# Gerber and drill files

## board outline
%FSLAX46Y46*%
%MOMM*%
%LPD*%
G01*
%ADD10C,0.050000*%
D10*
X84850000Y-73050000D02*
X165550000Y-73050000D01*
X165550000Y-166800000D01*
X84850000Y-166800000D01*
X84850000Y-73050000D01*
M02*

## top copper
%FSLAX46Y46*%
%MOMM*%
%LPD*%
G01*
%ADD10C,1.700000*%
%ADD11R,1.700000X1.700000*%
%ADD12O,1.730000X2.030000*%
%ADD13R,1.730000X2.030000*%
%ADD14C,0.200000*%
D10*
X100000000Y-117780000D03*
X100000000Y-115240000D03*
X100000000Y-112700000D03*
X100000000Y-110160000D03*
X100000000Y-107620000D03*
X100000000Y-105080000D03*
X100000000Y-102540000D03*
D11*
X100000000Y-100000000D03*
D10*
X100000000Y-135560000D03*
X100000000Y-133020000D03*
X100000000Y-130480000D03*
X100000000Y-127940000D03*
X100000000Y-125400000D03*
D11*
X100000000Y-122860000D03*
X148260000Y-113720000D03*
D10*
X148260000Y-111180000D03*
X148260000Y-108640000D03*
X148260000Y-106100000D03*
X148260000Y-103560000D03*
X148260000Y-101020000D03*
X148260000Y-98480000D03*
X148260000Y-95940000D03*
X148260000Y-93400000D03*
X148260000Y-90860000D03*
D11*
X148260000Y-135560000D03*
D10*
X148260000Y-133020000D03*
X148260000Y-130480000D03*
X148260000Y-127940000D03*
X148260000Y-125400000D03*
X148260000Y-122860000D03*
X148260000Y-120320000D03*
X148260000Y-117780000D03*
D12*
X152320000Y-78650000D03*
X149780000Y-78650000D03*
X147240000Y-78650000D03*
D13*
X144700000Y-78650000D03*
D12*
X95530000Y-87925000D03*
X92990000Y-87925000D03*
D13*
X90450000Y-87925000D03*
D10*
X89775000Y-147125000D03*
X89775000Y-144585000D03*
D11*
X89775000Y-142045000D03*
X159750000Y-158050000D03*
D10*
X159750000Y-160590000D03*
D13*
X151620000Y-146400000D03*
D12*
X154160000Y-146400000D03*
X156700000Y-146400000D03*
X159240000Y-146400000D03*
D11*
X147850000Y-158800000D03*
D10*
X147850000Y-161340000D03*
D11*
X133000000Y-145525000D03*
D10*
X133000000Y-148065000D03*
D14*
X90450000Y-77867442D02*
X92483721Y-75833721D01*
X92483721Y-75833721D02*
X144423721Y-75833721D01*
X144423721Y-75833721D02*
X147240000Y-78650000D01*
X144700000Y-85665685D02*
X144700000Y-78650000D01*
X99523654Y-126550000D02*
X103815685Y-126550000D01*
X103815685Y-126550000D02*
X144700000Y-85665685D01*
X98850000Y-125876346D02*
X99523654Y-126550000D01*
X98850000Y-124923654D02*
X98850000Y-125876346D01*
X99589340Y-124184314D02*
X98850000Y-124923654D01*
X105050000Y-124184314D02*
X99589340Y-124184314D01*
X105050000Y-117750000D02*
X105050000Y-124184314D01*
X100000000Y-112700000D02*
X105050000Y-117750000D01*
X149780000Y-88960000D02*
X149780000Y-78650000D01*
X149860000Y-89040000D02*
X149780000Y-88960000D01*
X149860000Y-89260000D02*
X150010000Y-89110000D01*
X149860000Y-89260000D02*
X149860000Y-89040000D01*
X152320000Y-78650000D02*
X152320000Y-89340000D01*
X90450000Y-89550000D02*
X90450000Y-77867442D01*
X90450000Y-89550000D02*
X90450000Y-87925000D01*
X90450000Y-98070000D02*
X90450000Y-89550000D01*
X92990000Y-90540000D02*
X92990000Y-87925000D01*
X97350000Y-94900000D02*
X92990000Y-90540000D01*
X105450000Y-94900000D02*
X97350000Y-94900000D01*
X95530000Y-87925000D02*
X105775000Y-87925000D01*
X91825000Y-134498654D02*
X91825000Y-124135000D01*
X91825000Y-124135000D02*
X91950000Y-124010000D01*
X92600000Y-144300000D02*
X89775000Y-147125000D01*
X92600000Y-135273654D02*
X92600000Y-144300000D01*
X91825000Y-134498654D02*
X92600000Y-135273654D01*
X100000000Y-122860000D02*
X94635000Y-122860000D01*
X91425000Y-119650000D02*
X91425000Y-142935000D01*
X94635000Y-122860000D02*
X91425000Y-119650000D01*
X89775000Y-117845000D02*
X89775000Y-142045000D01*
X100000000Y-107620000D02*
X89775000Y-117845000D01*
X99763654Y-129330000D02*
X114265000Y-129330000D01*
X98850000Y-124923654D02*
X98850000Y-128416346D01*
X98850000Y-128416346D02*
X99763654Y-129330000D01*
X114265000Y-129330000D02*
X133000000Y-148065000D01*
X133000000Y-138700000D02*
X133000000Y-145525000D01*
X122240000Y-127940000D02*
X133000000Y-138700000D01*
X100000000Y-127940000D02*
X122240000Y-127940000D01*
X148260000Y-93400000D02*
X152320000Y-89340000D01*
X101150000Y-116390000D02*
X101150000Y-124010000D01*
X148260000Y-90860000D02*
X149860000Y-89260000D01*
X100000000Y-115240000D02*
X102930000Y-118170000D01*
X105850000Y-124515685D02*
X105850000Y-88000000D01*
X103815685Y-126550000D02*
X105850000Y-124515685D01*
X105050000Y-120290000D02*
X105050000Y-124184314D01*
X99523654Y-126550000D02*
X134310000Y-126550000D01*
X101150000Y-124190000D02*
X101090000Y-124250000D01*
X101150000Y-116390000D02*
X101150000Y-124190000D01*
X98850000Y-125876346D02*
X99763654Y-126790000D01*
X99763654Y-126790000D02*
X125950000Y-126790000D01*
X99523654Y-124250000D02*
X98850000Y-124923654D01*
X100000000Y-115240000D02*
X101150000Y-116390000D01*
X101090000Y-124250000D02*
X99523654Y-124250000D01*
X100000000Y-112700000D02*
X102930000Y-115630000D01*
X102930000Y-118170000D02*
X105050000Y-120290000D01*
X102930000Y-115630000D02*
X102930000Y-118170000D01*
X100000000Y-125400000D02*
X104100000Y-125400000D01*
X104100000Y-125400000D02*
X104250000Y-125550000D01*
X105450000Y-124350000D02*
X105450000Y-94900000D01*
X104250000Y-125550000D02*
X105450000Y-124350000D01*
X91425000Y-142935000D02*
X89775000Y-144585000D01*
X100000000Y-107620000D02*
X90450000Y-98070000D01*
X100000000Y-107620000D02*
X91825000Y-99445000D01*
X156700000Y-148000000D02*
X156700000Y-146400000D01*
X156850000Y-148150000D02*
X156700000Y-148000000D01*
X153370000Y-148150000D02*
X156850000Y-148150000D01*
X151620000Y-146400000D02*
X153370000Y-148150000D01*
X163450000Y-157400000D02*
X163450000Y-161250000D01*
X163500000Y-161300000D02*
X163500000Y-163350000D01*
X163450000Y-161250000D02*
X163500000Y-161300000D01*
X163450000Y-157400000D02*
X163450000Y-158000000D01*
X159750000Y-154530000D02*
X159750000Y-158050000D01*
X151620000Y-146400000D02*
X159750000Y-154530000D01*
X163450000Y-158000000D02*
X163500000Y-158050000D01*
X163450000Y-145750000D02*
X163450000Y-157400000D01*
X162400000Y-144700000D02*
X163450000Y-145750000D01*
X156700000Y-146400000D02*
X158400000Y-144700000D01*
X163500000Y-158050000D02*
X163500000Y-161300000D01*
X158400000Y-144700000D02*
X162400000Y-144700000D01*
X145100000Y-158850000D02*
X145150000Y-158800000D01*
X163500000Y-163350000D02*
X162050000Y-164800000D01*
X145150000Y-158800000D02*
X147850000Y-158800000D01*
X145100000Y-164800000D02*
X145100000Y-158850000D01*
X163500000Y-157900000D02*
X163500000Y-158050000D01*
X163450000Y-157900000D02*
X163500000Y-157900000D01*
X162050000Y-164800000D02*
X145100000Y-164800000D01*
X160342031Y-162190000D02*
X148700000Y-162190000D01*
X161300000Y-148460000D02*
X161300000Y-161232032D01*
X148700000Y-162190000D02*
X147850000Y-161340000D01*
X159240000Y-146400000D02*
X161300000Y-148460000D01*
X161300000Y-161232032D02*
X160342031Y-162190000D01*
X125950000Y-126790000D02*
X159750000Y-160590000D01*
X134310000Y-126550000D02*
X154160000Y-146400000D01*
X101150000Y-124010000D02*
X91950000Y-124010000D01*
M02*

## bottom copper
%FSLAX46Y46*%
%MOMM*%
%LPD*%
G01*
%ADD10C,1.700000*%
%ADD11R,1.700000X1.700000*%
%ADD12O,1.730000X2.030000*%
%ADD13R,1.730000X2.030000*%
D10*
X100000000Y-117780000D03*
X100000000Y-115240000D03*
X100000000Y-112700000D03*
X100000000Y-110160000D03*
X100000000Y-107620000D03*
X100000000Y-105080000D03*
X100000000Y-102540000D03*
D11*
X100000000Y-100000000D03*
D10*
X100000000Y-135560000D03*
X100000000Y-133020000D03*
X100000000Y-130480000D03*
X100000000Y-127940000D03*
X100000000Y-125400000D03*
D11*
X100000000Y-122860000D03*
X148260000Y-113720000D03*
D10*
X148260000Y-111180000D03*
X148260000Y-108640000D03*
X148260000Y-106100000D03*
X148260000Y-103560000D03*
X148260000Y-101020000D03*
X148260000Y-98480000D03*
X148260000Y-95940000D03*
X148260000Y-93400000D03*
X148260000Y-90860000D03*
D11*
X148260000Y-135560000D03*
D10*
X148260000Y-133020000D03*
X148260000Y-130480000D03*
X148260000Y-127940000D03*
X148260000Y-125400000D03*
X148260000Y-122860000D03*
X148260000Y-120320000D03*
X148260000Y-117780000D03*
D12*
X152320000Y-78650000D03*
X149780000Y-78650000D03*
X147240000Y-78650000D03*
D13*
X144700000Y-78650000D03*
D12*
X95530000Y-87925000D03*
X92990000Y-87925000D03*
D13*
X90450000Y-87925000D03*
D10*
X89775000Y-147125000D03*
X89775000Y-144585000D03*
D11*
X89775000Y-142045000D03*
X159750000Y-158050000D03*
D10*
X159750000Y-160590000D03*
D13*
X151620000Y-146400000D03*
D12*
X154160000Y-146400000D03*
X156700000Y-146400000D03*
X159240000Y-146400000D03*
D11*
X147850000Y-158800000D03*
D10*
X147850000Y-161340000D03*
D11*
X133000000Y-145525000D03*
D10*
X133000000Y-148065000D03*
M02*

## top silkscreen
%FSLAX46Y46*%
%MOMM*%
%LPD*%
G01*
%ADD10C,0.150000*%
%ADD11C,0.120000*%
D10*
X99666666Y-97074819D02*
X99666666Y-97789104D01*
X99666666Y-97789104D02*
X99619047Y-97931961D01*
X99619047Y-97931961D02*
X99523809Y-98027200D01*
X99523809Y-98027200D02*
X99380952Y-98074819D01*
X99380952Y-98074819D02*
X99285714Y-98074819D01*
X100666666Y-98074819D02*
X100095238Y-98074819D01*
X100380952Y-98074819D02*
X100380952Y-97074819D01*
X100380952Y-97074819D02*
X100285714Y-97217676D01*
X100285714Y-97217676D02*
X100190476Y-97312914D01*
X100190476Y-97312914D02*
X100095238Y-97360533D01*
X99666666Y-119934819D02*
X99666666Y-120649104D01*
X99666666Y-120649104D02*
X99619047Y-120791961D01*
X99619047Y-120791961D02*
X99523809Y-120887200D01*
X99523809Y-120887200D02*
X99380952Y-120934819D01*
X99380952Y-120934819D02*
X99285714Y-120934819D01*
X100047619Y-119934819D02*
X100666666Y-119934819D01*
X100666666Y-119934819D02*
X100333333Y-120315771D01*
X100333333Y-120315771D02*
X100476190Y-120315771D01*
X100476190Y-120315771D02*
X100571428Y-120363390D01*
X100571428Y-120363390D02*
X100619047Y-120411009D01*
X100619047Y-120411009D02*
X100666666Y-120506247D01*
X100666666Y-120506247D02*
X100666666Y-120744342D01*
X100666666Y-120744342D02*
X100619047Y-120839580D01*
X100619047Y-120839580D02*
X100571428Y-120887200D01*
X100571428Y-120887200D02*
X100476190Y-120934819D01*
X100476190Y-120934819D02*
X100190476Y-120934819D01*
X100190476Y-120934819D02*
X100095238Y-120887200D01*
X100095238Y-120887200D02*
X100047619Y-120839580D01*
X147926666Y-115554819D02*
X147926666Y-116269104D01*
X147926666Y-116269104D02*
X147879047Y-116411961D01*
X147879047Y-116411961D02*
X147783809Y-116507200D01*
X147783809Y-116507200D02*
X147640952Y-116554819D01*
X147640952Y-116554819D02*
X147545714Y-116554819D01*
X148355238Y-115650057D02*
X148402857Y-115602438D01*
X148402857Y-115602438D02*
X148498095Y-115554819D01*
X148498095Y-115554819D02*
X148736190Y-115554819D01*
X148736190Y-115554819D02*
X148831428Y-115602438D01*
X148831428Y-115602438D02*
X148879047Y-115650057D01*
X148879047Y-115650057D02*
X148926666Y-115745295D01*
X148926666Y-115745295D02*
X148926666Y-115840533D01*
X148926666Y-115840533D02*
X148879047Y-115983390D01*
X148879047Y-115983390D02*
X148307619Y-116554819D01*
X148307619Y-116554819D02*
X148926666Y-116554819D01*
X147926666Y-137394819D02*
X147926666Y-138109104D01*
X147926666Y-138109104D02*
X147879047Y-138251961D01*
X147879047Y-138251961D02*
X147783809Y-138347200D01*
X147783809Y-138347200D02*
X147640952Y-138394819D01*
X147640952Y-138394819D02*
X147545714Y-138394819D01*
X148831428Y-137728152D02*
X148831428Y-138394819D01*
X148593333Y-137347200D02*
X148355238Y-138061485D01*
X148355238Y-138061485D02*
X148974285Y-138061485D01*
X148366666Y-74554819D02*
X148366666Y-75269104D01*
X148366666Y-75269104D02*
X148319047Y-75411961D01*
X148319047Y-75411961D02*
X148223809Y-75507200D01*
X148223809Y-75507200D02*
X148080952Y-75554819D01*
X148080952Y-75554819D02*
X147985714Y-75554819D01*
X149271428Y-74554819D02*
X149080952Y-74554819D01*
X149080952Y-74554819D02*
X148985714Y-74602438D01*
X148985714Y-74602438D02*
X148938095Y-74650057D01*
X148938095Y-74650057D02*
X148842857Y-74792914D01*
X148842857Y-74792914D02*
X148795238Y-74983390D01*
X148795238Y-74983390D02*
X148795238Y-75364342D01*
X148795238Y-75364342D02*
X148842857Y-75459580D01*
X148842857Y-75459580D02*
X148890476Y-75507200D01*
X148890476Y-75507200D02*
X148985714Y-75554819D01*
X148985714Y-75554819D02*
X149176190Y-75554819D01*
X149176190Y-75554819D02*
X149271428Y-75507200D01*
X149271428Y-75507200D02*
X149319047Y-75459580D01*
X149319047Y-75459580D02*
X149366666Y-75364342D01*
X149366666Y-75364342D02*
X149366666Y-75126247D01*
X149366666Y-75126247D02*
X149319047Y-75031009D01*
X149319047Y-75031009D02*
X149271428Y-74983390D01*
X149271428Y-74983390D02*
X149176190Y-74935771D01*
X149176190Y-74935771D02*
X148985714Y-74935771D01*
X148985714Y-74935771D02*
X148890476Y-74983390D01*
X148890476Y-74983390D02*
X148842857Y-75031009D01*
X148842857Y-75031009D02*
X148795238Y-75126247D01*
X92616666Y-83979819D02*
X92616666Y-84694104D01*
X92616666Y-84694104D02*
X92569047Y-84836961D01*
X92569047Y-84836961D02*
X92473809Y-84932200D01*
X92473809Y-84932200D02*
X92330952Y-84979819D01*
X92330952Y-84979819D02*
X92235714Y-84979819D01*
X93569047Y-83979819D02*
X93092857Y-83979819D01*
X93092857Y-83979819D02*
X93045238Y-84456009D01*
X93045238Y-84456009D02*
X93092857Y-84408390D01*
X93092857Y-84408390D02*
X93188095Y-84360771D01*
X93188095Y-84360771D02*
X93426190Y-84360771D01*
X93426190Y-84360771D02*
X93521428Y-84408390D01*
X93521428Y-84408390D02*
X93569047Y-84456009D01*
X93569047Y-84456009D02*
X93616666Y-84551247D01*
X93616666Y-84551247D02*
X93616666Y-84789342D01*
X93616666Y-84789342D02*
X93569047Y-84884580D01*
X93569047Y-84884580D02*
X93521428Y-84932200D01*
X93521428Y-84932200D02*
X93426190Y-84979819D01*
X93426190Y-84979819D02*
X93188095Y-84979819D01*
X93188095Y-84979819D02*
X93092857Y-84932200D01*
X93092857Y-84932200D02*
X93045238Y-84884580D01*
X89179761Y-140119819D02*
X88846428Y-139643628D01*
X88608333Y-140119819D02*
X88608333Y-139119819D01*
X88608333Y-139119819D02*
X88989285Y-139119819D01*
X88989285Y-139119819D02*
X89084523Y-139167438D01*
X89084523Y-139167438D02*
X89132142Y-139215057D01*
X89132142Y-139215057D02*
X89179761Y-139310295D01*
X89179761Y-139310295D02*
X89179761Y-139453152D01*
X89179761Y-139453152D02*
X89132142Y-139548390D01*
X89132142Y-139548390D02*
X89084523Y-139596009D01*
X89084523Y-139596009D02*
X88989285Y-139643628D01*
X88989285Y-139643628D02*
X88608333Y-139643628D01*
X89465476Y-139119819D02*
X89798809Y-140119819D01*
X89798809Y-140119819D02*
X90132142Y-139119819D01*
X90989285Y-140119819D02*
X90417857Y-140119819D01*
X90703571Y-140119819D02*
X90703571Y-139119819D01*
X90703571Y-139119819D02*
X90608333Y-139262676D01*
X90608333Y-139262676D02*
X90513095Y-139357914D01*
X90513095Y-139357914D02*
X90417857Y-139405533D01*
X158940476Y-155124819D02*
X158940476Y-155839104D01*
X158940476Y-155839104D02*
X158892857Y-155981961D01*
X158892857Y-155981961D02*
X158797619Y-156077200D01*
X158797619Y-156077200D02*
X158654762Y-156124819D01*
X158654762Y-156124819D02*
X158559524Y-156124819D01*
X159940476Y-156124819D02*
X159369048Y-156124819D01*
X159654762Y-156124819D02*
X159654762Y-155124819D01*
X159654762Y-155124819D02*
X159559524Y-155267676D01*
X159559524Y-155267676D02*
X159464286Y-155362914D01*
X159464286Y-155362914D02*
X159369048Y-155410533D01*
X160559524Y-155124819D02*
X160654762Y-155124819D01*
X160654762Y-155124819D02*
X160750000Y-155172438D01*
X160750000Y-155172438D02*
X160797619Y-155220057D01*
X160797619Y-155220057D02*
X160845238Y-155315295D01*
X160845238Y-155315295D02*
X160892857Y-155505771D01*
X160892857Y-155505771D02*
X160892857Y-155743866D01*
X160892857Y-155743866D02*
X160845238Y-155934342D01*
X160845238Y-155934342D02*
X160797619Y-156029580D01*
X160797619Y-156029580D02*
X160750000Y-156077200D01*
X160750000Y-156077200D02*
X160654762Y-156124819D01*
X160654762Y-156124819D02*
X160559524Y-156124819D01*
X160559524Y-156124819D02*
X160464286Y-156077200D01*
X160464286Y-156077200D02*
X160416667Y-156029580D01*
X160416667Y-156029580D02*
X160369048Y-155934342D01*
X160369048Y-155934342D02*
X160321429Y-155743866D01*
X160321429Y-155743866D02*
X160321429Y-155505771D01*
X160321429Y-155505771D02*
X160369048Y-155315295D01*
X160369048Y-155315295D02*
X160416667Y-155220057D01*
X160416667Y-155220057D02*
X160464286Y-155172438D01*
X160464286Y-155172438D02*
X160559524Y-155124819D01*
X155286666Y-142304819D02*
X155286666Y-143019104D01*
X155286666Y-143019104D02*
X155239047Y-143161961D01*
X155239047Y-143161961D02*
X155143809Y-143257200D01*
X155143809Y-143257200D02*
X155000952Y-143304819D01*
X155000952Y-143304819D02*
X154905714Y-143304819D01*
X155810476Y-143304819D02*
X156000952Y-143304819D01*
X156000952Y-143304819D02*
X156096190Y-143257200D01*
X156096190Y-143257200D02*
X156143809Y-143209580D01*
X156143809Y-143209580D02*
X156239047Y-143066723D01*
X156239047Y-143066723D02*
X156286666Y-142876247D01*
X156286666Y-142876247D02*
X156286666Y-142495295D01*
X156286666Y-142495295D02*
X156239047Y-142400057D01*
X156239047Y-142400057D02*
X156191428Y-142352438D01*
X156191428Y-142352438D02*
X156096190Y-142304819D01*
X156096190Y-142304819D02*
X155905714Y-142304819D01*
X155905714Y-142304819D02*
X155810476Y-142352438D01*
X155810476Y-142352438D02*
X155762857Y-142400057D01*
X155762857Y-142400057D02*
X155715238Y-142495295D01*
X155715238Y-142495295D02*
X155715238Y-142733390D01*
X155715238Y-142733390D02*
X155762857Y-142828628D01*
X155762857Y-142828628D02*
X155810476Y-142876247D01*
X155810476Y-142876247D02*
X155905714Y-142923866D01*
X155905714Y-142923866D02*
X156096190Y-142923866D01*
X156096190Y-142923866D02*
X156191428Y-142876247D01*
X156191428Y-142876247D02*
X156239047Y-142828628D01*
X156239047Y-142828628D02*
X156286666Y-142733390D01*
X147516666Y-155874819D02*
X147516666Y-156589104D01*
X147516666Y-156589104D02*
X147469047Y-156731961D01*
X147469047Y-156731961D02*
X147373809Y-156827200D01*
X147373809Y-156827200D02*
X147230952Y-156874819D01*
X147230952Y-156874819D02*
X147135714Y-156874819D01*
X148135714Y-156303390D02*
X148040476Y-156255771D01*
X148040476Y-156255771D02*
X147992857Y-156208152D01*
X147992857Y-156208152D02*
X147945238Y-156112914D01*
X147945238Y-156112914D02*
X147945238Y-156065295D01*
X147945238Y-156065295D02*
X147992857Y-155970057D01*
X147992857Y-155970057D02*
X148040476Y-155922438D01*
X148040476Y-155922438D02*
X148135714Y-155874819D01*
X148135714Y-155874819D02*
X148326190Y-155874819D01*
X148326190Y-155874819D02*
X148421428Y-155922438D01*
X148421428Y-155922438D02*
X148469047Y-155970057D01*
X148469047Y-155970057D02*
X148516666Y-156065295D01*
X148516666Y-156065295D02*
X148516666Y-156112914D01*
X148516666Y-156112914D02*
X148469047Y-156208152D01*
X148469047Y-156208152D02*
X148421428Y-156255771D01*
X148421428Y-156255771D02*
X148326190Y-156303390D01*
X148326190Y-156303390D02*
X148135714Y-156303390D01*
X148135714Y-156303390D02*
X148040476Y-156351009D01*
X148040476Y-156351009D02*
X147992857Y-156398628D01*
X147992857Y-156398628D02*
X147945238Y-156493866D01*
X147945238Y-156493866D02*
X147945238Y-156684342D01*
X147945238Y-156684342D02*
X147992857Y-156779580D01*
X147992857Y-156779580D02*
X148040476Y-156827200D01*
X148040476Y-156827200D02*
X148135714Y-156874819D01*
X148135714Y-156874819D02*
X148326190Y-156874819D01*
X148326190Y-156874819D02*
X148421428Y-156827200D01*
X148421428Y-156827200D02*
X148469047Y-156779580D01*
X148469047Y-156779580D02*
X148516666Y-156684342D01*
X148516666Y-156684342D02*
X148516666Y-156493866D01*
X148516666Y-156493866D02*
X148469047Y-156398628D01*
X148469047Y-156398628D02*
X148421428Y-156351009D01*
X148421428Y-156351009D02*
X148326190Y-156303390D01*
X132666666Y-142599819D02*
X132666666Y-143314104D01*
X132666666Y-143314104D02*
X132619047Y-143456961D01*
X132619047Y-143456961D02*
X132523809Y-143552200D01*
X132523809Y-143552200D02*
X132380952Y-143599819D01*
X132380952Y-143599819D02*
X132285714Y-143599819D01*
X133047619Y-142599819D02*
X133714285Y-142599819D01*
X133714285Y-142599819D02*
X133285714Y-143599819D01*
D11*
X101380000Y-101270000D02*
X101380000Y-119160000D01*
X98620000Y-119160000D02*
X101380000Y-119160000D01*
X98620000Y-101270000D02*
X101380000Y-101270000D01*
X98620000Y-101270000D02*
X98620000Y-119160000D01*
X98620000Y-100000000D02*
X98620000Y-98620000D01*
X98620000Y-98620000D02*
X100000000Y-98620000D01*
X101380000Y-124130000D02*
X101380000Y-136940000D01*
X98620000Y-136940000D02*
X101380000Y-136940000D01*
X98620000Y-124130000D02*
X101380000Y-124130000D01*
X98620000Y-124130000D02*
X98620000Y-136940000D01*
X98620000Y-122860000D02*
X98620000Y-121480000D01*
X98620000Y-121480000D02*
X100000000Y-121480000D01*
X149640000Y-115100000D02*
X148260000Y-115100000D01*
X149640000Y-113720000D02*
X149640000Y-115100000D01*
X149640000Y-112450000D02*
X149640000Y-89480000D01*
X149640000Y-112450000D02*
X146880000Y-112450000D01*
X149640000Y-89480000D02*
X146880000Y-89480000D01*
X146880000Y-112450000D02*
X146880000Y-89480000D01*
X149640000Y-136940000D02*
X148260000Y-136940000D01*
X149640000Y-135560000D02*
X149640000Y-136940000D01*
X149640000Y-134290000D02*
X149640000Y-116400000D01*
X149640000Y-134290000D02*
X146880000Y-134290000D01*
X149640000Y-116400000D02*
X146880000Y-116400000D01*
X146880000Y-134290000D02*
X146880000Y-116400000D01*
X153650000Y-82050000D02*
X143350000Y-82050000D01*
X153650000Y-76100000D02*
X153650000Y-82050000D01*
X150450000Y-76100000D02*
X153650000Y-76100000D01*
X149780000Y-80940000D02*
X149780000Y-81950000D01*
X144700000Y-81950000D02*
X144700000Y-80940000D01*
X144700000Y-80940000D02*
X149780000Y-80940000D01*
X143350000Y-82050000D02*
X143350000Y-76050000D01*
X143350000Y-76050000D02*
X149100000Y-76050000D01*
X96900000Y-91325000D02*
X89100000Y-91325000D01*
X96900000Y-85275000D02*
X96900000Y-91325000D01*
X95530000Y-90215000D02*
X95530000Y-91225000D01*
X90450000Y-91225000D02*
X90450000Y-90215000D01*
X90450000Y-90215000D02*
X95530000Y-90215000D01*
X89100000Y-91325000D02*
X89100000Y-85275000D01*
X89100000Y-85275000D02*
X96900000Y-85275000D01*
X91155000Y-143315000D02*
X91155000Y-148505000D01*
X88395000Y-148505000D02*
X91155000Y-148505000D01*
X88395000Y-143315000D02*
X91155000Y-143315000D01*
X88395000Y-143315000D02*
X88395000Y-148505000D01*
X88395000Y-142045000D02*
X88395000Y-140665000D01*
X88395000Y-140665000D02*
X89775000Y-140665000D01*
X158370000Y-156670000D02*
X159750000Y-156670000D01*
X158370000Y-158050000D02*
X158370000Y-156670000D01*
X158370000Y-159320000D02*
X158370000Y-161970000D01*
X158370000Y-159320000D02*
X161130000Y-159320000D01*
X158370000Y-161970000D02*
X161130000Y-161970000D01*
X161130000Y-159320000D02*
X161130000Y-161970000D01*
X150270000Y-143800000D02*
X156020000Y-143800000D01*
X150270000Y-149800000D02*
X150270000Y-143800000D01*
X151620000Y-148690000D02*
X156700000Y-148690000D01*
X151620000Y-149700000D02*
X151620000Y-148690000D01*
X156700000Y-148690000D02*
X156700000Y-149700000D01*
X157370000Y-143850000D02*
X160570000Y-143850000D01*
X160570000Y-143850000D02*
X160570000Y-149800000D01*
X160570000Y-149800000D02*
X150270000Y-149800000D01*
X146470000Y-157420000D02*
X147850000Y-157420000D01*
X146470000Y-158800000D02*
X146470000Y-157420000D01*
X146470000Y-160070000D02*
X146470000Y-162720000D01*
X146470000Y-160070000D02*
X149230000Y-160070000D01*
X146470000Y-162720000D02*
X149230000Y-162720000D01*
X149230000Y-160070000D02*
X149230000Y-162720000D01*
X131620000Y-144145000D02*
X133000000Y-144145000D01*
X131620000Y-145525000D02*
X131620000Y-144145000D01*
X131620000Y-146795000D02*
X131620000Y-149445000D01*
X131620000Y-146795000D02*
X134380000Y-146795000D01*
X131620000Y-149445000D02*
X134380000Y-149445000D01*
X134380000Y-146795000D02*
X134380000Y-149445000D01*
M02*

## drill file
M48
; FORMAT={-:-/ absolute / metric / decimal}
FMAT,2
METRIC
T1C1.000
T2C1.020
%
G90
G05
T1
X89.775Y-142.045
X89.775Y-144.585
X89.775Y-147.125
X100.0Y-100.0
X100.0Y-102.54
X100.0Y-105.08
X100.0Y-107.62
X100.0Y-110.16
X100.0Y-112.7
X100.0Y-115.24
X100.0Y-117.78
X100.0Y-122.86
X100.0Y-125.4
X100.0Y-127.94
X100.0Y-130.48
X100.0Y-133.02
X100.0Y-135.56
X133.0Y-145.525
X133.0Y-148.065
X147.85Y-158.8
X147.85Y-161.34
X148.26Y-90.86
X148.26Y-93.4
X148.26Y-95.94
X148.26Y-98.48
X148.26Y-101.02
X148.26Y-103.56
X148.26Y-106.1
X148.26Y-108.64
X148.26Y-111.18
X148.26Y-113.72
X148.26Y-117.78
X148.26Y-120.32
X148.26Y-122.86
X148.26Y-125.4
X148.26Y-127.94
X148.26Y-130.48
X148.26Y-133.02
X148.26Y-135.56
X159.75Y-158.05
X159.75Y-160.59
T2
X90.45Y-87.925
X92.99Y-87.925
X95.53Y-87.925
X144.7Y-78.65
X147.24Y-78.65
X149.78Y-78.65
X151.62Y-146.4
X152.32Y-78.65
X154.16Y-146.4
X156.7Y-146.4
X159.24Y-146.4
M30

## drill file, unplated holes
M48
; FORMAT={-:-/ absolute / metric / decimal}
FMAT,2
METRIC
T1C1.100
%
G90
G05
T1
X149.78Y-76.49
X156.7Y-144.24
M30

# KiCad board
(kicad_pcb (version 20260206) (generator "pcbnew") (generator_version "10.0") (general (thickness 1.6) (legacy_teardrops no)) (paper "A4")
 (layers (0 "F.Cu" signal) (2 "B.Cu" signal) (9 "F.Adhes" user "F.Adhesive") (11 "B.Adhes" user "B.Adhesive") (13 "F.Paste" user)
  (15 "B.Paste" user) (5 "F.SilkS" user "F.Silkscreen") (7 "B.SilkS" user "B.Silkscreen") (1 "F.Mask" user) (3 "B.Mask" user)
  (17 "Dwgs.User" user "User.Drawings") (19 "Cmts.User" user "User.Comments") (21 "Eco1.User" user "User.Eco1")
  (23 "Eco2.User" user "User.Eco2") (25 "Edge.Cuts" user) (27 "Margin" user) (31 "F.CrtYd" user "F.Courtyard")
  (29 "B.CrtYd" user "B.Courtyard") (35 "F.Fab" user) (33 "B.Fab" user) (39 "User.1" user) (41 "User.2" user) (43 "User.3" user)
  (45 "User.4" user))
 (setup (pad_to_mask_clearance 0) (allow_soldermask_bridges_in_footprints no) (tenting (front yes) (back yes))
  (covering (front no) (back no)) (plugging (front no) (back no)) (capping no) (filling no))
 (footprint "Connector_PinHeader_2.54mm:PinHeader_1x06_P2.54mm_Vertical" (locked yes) (layer "F.Cu") (at 100 122.86)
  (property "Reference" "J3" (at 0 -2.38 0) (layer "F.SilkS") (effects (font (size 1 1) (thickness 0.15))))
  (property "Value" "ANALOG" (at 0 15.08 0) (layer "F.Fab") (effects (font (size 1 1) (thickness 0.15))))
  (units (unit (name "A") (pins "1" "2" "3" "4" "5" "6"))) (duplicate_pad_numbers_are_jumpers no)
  (fp_line (start -1.38 -1.38) (end 0 -1.38) (stroke (width 0.12) (type solid)) (layer "F.SilkS"))
  (fp_line (start -1.38 0) (end -1.38 -1.38) (stroke (width 0.12) (type solid)) (layer "F.SilkS"))
  (fp_line (start -1.38 1.27) (end -1.38 14.08) (stroke (width 0.12) (type solid)) (layer "F.SilkS"))
  (fp_line (start -1.38 1.27) (end 1.38 1.27) (stroke (width 0.12) (type solid)) (layer "F.SilkS"))
  (fp_line (start -1.38 14.08) (end 1.38 14.08) (stroke (width 0.12) (type solid)) (layer "F.SilkS"))
  (fp_line (start 1.38 1.27) (end 1.38 14.08) (stroke (width 0.12) (type solid)) (layer "F.SilkS"))
  (pad "1" thru_hole rect (at 0 0) (size 1.7 1.7) (drill 1) (layers "*.Cu" "*.Mask") (remove_unused_layers no) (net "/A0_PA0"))
  (pad "2" thru_hole circle (at 0 2.54) (size 1.7 1.7) (drill 1) (layers "*.Cu" "*.Mask") (remove_unused_layers no) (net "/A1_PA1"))
  (pad "3" thru_hole circle (at 0 5.08) (size 1.7 1.7) (drill 1) (layers "*.Cu" "*.Mask") (remove_unused_layers no) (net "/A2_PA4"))
  (pad "4" thru_hole circle (at 0 7.62) (size 1.7 1.7) (drill 1) (layers "*.Cu" "*.Mask") (remove_unused_layers no)
   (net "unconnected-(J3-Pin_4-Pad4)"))
  (pad "5" thru_hole circle (at 0 10.16) (size 1.7 1.7) (drill 1) (layers "*.Cu" "*.Mask") (remove_unused_layers no)
   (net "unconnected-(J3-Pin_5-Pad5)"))
  (pad "6" thru_hole circle (at 0 12.7) (size 1.7 1.7) (drill 1) (layers "*.Cu" "*.Mask") (remove_unused_layers no)
   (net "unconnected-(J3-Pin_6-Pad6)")))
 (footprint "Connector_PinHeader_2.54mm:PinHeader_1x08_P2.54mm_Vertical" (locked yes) (layer "F.Cu") (at 100 100)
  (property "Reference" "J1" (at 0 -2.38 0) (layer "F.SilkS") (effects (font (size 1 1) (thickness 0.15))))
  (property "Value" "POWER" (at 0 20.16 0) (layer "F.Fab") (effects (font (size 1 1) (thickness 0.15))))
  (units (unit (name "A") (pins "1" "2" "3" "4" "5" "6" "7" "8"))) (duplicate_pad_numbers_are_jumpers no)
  (fp_line (start -1.38 -1.38) (end 0 -1.38) (stroke (width 0.12) (type solid)) (layer "F.SilkS"))
  (fp_line (start -1.38 0) (end -1.38 -1.38) (stroke (width 0.12) (type solid)) (layer "F.SilkS"))
  (fp_line (start -1.38 1.27) (end -1.38 19.16) (stroke (width 0.12) (type solid)) (layer "F.SilkS"))
  (fp_line (start -1.38 1.27) (end 1.38 1.27) (stroke (width 0.12) (type solid)) (layer "F.SilkS"))
  (fp_line (start -1.38 19.16) (end 1.38 19.16) (stroke (width 0.12) (type solid)) (layer "F.SilkS"))
  (fp_line (start 1.38 1.27) (end 1.38 19.16) (stroke (width 0.12) (type solid)) (layer "F.SilkS"))
  (pad "1" thru_hole rect (at 0 0) (size 1.7 1.7) (drill 1) (layers "*.Cu" "*.Mask") (remove_unused_layers no) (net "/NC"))
  (pad "2" thru_hole circle (at 0 2.54) (size 1.7 1.7) (drill 1) (layers "*.Cu" "*.Mask") (remove_unused_layers no) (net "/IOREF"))
  (pad "3" thru_hole circle (at 0 5.08) (size 1.7 1.7) (drill 1) (layers "*.Cu" "*.Mask") (remove_unused_layers no) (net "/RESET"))
  (pad "4" thru_hole circle (at 0 7.62) (size 1.7 1.7) (drill 1) (layers "*.Cu" "*.Mask") (remove_unused_layers no) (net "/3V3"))
  (pad "5" thru_hole circle (at 0 10.16) (size 1.7 1.7) (drill 1) (layers "*.Cu" "*.Mask") (remove_unused_layers no) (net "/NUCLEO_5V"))
  (pad "6" thru_hole circle (at 0 12.7) (size 1.7 1.7) (drill 1) (layers "*.Cu" "*.Mask") (remove_unused_layers no) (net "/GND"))
  (pad "7" thru_hole circle (at 0 15.24) (size 1.7 1.7) (drill 1) (layers "*.Cu" "*.Mask") (remove_unused_layers no) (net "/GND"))
  (pad "8" thru_hole circle (at 0 17.78) (size 1.7 1.7) (drill 1) (layers "*.Cu" "*.Mask") (remove_unused_layers no) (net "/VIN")))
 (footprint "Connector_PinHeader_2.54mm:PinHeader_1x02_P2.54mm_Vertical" (layer "F.Cu") (at 159.75 158.05)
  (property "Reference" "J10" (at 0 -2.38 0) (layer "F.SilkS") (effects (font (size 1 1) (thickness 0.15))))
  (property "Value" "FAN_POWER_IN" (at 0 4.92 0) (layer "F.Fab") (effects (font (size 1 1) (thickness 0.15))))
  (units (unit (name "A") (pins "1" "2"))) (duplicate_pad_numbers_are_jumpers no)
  (fp_line (start -1.38 -1.38) (end 0 -1.38) (stroke (width 0.12) (type solid)) (layer "F.SilkS"))
  (fp_line (start -1.38 0) (end -1.38 -1.38) (stroke (width 0.12) (type solid)) (layer "F.SilkS"))
  (fp_line (start -1.38 1.27) (end -1.38 3.92) (stroke (width 0.12) (type solid)) (layer "F.SilkS"))
  (fp_line (start -1.38 1.27) (end 1.38 1.27) (stroke (width 0.12) (type solid)) (layer "F.SilkS"))
  (fp_line (start -1.38 3.92) (end 1.38 3.92) (stroke (width 0.12) (type solid)) (layer "F.SilkS"))
  (fp_line (start 1.38 1.27) (end 1.38 3.92) (stroke (width 0.12) (type solid)) (layer "F.SilkS"))
  (pad "1" thru_hole rect (at 0 0) (size 1.7 1.7) (drill 1) (layers "*.Cu" "*.Mask") (remove_unused_layers no) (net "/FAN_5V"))
  (pad "2" thru_hole circle (at 0 2.54) (size 1.7 1.7) (drill 1) (layers "*.Cu" "*.Mask") (remove_unused_layers no) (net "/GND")))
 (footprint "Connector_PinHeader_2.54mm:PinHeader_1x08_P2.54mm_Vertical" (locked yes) (layer "F.Cu") (at 148.26 135.56 180)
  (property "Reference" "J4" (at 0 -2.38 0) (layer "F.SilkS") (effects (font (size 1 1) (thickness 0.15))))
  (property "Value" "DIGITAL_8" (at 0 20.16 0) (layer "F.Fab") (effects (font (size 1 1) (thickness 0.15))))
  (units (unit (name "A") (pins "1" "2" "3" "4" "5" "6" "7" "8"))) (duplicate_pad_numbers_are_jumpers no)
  (fp_line (start 1.38 1.27) (end 1.38 19.16) (stroke (width 0.12) (type solid)) (layer "F.SilkS"))
  (fp_line (start -1.38 19.16) (end 1.38 19.16) (stroke (width 0.12) (type solid)) (layer "F.SilkS"))
  (fp_line (start -1.38 1.27) (end 1.38 1.27) (stroke (width 0.12) (type solid)) (layer "F.SilkS"))
  (fp_line (start -1.38 1.27) (end -1.38 19.16) (stroke (width 0.12) (type solid)) (layer "F.SilkS"))
  (fp_line (start -1.38 0) (end -1.38 -1.38) (stroke (width 0.12) (type solid)) (layer "F.SilkS"))
  (fp_line (start -1.38 -1.38) (end 0 -1.38) (stroke (width 0.12) (type solid)) (layer "F.SilkS"))
  (pad "1" thru_hole rect (at 0 0 180) (size 1.7 1.7) (drill 1) (layers "*.Cu" "*.Mask") (remove_unused_layers no) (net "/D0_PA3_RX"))
  (pad "2" thru_hole circle (at 0 2.54 180) (size 1.7 1.7) (drill 1) (layers "*.Cu" "*.Mask") (remove_unused_layers no) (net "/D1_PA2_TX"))
  (pad "3" thru_hole circle (at 0 5.08 180) (size 1.7 1.7) (drill 1) (layers "*.Cu" "*.Mask") (remove_unused_layers no) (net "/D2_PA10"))
  (pad "4" thru_hole circle (at 0 7.62 180) (size 1.7 1.7) (drill 1) (layers "*.Cu" "*.Mask") (remove_unused_layers no) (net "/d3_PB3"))
  (pad "5" thru_hole circle (at 0 10.16 180) (size 1.7 1.7) (drill 1) (layers "*.Cu" "*.Mask") (remove_unused_layers no) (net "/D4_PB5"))
  (pad "6" thru_hole circle (at 0 12.7 180) (size 1.7 1.7) (drill 1) (layers "*.Cu" "*.Mask") (remove_unused_layers no) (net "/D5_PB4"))
  (pad "7" thru_hole circle (at 0 15.24 180) (size 1.7 1.7) (drill 1) (layers "*.Cu" "*.Mask") (remove_unused_layers no) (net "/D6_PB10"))
  (pad "8" thru_hole circle (at 0 17.78 180) (size 1.7 1.7) (drill 1) (layers "*.Cu" "*.Mask") (remove_unused_layers no) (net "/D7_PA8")))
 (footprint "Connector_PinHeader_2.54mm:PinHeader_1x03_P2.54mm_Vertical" (layer "F.Cu") (at 89.775 142.045)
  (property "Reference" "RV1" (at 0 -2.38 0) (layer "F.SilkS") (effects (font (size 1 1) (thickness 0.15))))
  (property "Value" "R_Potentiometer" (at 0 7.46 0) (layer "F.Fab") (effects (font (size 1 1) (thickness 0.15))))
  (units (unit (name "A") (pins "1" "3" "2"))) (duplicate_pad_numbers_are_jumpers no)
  (fp_line (start -1.38 -1.38) (end 0 -1.38) (stroke (width 0.12) (type solid)) (layer "F.SilkS"))
  (fp_line (start -1.38 0) (end -1.38 -1.38) (stroke (width 0.12) (type solid)) (layer "F.SilkS"))
  (fp_line (start -1.38 1.27) (end -1.38 6.46) (stroke (width 0.12) (type solid)) (layer "F.SilkS"))
  (fp_line (start -1.38 1.27) (end 1.38 1.27) (stroke (width 0.12) (type solid)) (layer "F.SilkS"))
  (fp_line (start -1.38 6.46) (end 1.38 6.46) (stroke (width 0.12) (type solid)) (layer "F.SilkS"))
  (fp_line (start 1.38 1.27) (end 1.38 6.46) (stroke (width 0.12) (type solid)) (layer "F.SilkS"))
  (pad "1" thru_hole rect (at 0 0) (size 1.7 1.7) (drill 1) (layers "*.Cu" "*.Mask") (remove_unused_layers no) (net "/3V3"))
  (pad "2" thru_hole circle (at 0 2.54) (size 1.7 1.7) (drill 1) (layers "*.Cu" "*.Mask") (remove_unused_layers no) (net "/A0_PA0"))
  (pad "3" thru_hole circle (at 0 5.08) (size 1.7 1.7) (drill 1) (layers "*.Cu" "*.Mask") (remove_unused_layers no) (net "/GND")))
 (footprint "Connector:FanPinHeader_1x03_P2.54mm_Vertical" (layer "F.Cu") (at 90.45 87.925)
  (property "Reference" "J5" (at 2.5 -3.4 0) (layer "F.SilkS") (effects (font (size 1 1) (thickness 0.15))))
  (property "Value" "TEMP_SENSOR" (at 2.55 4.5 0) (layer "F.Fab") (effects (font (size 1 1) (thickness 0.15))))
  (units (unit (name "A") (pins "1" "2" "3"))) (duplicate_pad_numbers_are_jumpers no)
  (fp_line (start -1.35 -2.65) (end 6.45 -2.65) (stroke (width 0.12) (type solid)) (layer "F.SilkS"))
  (fp_line (start -1.35 3.4) (end -1.35 -2.65) (stroke (width 0.12) (type solid)) (layer "F.SilkS"))
  (fp_line (start 0 2.29) (end 5.08 2.29) (stroke (width 0.12) (type solid)) (layer "F.SilkS"))
  (fp_line (start 0 3.3) (end 0 2.29) (stroke (width 0.12) (type solid)) (layer "F.SilkS"))
  (fp_line (start 5.08 2.29) (end 5.08 3.3) (stroke (width 0.12) (type solid)) (layer "F.SilkS"))
  (fp_line (start 6.45 -2.65) (end 6.45 3.4) (stroke (width 0.12) (type solid)) (layer "F.SilkS"))
  (fp_line (start 6.45 3.4) (end -1.35 3.4) (stroke (width 0.12) (type solid)) (layer "F.SilkS"))
  (pad "1" thru_hole rect (at 0 0 90) (size 2.03 1.73) (drill 1.02) (layers "*.Cu" "*.Mask") (remove_unused_layers no) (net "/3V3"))
  (pad "2" thru_hole oval (at 2.54 0 90) (size 2.03 1.73) (drill 1.02) (layers "*.Cu" "*.Mask") (remove_unused_layers no) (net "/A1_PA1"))
  (pad "3" thru_hole oval (at 5.08 0 90) (size 2.03 1.73) (drill 1.02) (layers "*.Cu" "*.Mask") (remove_unused_layers no) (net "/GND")))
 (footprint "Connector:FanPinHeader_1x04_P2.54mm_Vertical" (layer "F.Cu") (at 151.62 146.4)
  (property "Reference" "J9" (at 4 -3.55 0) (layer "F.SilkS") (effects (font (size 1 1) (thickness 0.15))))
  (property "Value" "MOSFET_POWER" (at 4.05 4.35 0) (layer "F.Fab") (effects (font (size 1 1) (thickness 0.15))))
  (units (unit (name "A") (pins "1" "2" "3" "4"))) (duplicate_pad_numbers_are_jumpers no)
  (fp_line (start -1.35 -2.6) (end 4.4 -2.6) (stroke (width 0.12) (type solid)) (layer "F.SilkS"))
  (fp_line (start -1.35 3.4) (end -1.35 -2.6) (stroke (width 0.12) (type solid)) (layer "F.SilkS"))
  (fp_line (start 0 2.29) (end 5.08 2.29) (stroke (width 0.12) (type solid)) (layer "F.SilkS"))
  (fp_line (start 0 3.3) (end 0 2.29) (stroke (width 0.12) (type solid)) (layer "F.SilkS"))
  (fp_line (start 5.08 2.29) (end 5.08 3.3) (stroke (width 0.12) (type solid)) (layer "F.SilkS"))
  (fp_line (start 5.75 -2.55) (end 8.95 -2.55) (stroke (width 0.12) (type solid)) (layer "F.SilkS"))
  (fp_line (start 8.95 -2.55) (end 8.95 3.4) (stroke (width 0.12) (type solid)) (layer "F.SilkS"))
  (fp_line (start 8.95 3.4) (end -1.35 3.4) (stroke (width 0.12) (type solid)) (layer "F.SilkS"))
  (pad "" np_thru_hole circle (at 5.08 -2.16 90) (size 1.1 1.1) (drill 1.1) (layers "*.Cu" "*.Mask"))
  (pad "1" thru_hole rect (at 0 0 90) (size 2.03 1.73) (drill 1.02) (layers "*.Cu" "*.Mask") (remove_unused_layers no) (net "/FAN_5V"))
  (pad "2" thru_hole oval (at 2.54 0 90) (size 2.03 1.73) (drill 1.02) (layers "*.Cu" "*.Mask") (remove_unused_layers no) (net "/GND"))
  (pad "3" thru_hole oval (at 5.08 0 90) (size 2.03 1.73) (drill 1.02) (layers "*.Cu" "*.Mask") (remove_unused_layers no) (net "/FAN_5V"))
  (pad "4" thru_hole oval (at 7.62 0 90) (size 2.03 1.73) (drill 1.02) (layers "*.Cu" "*.Mask") (remove_unused_layers no) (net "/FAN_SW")))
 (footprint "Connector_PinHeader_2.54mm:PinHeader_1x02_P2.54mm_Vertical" (layer "F.Cu") (at 133 145.525)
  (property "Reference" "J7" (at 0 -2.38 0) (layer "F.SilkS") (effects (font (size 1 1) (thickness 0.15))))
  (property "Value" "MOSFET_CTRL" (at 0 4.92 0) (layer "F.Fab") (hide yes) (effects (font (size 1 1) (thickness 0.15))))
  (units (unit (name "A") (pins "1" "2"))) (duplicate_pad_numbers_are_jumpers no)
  (fp_line (start -1.38 -1.38) (end 0 -1.38) (stroke (width 0.12) (type solid)) (layer "F.SilkS"))
  (fp_line (start -1.38 0) (end -1.38 -1.38) (stroke (width 0.12) (type solid)) (layer "F.SilkS"))
  (fp_line (start -1.38 1.27) (end -1.38 3.92) (stroke (width 0.12) (type solid)) (layer "F.SilkS"))
  (fp_line (start -1.38 1.27) (end 1.38 1.27) (stroke (width 0.12) (type solid)) (layer "F.SilkS"))
  (fp_line (start -1.38 3.92) (end 1.38 3.92) (stroke (width 0.12) (type solid)) (layer "F.SilkS"))
  (fp_line (start 1.38 1.27) (end 1.38 3.92) (stroke (width 0.12) (type solid)) (layer "F.SilkS"))
  (pad "1" thru_hole rect (at 0 0) (size 1.7 1.7) (drill 1) (layers "*.Cu" "*.Mask") (remove_unused_layers no) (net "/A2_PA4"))
  (pad "2" thru_hole circle (at 0 2.54) (size 1.7 1.7) (drill 1) (layers "*.Cu" "*.Mask") (remove_unused_layers no) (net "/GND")))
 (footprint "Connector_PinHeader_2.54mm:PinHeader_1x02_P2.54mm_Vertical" (layer "F.Cu") (at 147.85 158.8)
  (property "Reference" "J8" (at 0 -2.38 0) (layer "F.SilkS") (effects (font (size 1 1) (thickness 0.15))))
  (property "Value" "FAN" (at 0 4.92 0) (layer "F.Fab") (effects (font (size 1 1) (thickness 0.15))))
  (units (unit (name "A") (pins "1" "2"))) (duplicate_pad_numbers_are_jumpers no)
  (fp_line (start -1.38 -1.38) (end 0 -1.38) (stroke (width 0.12) (type solid)) (layer "F.SilkS"))
  (fp_line (start -1.38 0) (end -1.38 -1.38) (stroke (width 0.12) (type solid)) (layer "F.SilkS"))
  (fp_line (start -1.38 1.27) (end -1.38 3.92) (stroke (width 0.12) (type solid)) (layer "F.SilkS"))
  (fp_line (start -1.38 1.27) (end 1.38 1.27) (stroke (width 0.12) (type solid)) (layer "F.SilkS"))
  (fp_line (start -1.38 3.92) (end 1.38 3.92) (stroke (width 0.12) (type solid)) (layer "F.SilkS"))
  (fp_line (start 1.38 1.27) (end 1.38 3.92) (stroke (width 0.12) (type solid)) (layer "F.SilkS"))
  (pad "1" thru_hole rect (at 0 0) (size 1.7 1.7) (drill 1) (layers "*.Cu" "*.Mask") (remove_unused_layers no) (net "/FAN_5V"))
  (pad "2" thru_hole circle (at 0 2.54) (size 1.7 1.7) (drill 1) (layers "*.Cu" "*.Mask") (remove_unused_layers no) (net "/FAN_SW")))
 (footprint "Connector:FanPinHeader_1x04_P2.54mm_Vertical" (layer "F.Cu") (at 144.7 78.65)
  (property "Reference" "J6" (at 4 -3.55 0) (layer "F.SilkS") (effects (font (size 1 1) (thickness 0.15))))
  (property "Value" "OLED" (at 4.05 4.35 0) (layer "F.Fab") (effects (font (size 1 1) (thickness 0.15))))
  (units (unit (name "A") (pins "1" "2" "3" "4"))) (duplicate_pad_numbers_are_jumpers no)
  (fp_line (start -1.35 -2.6) (end 4.4 -2.6) (stroke (width 0.12) (type solid)) (layer "F.SilkS"))
  (fp_line (start -1.35 3.4) (end -1.35 -2.6) (stroke (width 0.12) (type solid)) (layer "F.SilkS"))
  (fp_line (start 0 2.29) (end 5.08 2.29) (stroke (width 0.12) (type solid)) (layer "F.SilkS"))
  (fp_line (start 0 3.3) (end 0 2.29) (stroke (width 0.12) (type solid)) (layer "F.SilkS"))
  (fp_line (start 5.08 2.29) (end 5.08 3.3) (stroke (width 0.12) (type solid)) (layer "F.SilkS"))
  (fp_line (start 5.75 -2.55) (end 8.95 -2.55) (stroke (width 0.12) (type solid)) (layer "F.SilkS"))
  (fp_line (start 8.95 -2.55) (end 8.95 3.4) (stroke (width 0.12) (type solid)) (layer "F.SilkS"))
  (fp_line (start 8.95 3.4) (end -1.35 3.4) (stroke (width 0.12) (type solid)) (layer "F.SilkS"))
  (pad "" np_thru_hole circle (at 5.08 -2.16 90) (size 1.1 1.1) (drill 1.1) (layers "*.Cu" "*.Mask"))
  (pad "1" thru_hole rect (at 0 0 90) (size 2.03 1.73) (drill 1.02) (layers "*.Cu" "*.Mask") (remove_unused_layers no) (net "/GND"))
  (pad "2" thru_hole oval (at 2.54 0 90) (size 2.03 1.73) (drill 1.02) (layers "*.Cu" "*.Mask") (remove_unused_layers no) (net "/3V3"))
  (pad "3" thru_hole oval (at 5.08 0 90) (size 2.03 1.73) (drill 1.02) (layers "*.Cu" "*.Mask") (remove_unused_layers no)
   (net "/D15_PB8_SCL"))
  (pad "4" thru_hole oval (at 7.62 0 90) (size 2.03 1.73) (drill 1.02) (layers "*.Cu" "*.Mask") (remove_unused_layers no)
   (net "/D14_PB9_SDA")))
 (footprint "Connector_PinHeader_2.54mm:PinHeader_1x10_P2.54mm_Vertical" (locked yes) (layer "F.Cu") (at 148.26 113.72 180)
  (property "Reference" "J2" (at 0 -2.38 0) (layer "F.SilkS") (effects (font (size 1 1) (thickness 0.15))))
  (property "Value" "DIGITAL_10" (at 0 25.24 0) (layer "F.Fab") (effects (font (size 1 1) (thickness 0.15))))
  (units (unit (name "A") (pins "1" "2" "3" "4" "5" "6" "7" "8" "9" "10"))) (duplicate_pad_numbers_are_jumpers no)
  (fp_line (start 1.38 1.27) (end 1.38 24.24) (stroke (width 0.12) (type solid)) (layer "F.SilkS"))
  (fp_line (start -1.38 24.24) (end 1.38 24.24) (stroke (width 0.12) (type solid)) (layer "F.SilkS"))
  (fp_line (start -1.38 1.27) (end 1.38 1.27) (stroke (width 0.12) (type solid)) (layer "F.SilkS"))
  (fp_line (start -1.38 1.27) (end -1.38 24.24) (stroke (width 0.12) (type solid)) (layer "F.SilkS"))
  (fp_line (start -1.38 0) (end -1.38 -1.38) (stroke (width 0.12) (type solid)) (layer "F.SilkS"))
  (fp_line (start -1.38 -1.38) (end 0 -1.38) (stroke (width 0.12) (type solid)) (layer "F.SilkS"))
  (pad "1" thru_hole rect (at 0 0 180) (size 1.7 1.7) (drill 1) (layers "*.Cu" "*.Mask") (remove_unused_layers no)
   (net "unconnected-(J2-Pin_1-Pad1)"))
  (pad "2" thru_hole circle (at 0 2.54 180) (size 1.7 1.7) (drill 1) (layers "*.Cu" "*.Mask") (remove_unused_layers no)
   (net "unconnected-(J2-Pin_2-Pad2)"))
  (pad "3" thru_hole circle (at 0 5.08 180) (size 1.7 1.7) (drill 1) (layers "*.Cu" "*.Mask") (remove_unused_layers no)
   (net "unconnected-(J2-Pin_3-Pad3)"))
  (pad "4" thru_hole circle (at 0 7.62 180) (size 1.7 1.7) (drill 1) (layers "*.Cu" "*.Mask") (remove_unused_layers no)
   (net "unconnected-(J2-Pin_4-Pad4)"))
  (pad "5" thru_hole circle (at 0 10.16 180) (size 1.7 1.7) (drill 1) (layers "*.Cu" "*.Mask") (remove_unused_layers no)
   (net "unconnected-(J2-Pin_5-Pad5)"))
  (pad "6" thru_hole circle (at 0 12.7 180) (size 1.7 1.7) (drill 1) (layers "*.Cu" "*.Mask") (remove_unused_layers no)
   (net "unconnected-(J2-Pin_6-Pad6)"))
  (pad "7" thru_hole circle (at 0 15.24 180) (size 1.7 1.7) (drill 1) (layers "*.Cu" "*.Mask") (remove_unused_layers no)
   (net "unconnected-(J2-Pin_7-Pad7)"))
  (pad "8" thru_hole circle (at 0 17.78 180) (size 1.7 1.7) (drill 1) (layers "*.Cu" "*.Mask") (remove_unused_layers no)
   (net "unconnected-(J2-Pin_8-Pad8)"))
  (pad "9" thru_hole circle (at 0 20.32 180) (size 1.7 1.7) (drill 1) (layers "*.Cu" "*.Mask") (remove_unused_layers no)
   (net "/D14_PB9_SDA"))
  (pad "10" thru_hole circle (at 0 22.86 180) (size 1.7 1.7) (drill 1) (layers "*.Cu" "*.Mask") (remove_unused_layers no)
   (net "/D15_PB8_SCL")))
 (gr_rect (start 84.85 73.05) (end 165.55 166.8) (stroke (width 0.05) (type default)) (fill no) (layer "Edge.Cuts"))
 (segment (start 102.93 115.63) (end 102.93 118.17) (width 0.2) (layer "F.Cu") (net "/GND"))
 (segment (start 92.6 135.273654) (end 92.6 144.3) (width 0.2) (layer "F.Cu") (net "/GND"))
 (segment (start 134.31 126.55) (end 154.16 146.4) (width 0.2) (layer "F.Cu") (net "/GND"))
 (segment (start 100 112.7) (end 102.93 115.63) (width 0.2) (layer "F.Cu") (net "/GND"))
 (segment (start 103.815685 126.55) (end 144.7 85.665685) (width 0.2) (layer "F.Cu") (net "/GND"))
 (segment (start 99.763654 129.33) (end 114.265 129.33) (width 0.2) (layer "F.Cu") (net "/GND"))
 (segment (start 91.825 124.135) (end 91.95 124.01) (width 0.2) (layer "F.Cu") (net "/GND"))
 (segment (start 101.15 124.19) (end 101.09 124.25) (width 0.2) (layer "F.Cu") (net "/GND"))
 (segment (start 91.825 134.498654) (end 91.825 124.135) (width 0.2) (layer "F.Cu") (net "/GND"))
 (segment (start 105.05 120.29) (end 105.05 124.184314) (width 0.2) (layer "F.Cu") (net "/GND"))
 (segment (start 98.85 124.923654) (end 98.85 128.416346) (width 0.2) (layer "F.Cu") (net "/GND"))
 (segment (start 114.265 129.33) (end 133 148.065) (width 0.2) (layer "F.Cu") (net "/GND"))
 (segment (start 101.15 116.39) (end 101.15 124.19) (width 0.2) (layer "F.Cu") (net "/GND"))
 (segment (start 95.53 87.925) (end 105.775 87.925) (width 0.2) (layer "F.Cu") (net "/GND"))
 (segment (start 99.523654 126.55) (end 103.815685 126.55) (width 0.2) (layer "F.Cu") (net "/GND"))
 (segment (start 105.85 124.515685) (end 105.85 88) (width 0.2) (layer "F.Cu") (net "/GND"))
 (segment (start 101.15 116.39) (end 101.15 124.01) (width 0.2) (layer "F.Cu") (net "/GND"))
 (segment (start 125.95 126.79) (end 159.75 160.59) (width 0.2) (layer "F.Cu") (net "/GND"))
 (segment (start 98.85 125.876346) (end 99.763654 126.79) (width 0.2) (layer "F.Cu") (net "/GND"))
 (segment (start 92.6 144.3) (end 89.775 147.125) (width 0.2) (layer "F.Cu") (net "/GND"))
 (segment (start 99.523654 126.55) (end 134.31 126.55) (width 0.2) (layer "F.Cu") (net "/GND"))
 (segment (start 103.815685 126.55) (end 105.85 124.515685) (width 0.2) (layer "F.Cu") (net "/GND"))
 (segment (start 102.93 118.17) (end 105.05 120.29) (width 0.2) (layer "F.Cu") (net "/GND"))
 (segment (start 105.05 124.184314) (end 99.58934 124.184314) (width 0.2) (layer "F.Cu") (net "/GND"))
 (segment (start 99.523654 124.25) (end 98.85 124.923654) (width 0.2) (layer "F.Cu") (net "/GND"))
 (segment (start 98.85 125.876346) (end 99.523654 126.55) (width 0.2) (layer "F.Cu") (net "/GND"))
 (segment (start 100 112.7) (end 105.05 117.75) (width 0.2) (layer "F.Cu") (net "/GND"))
 (segment (start 99.58934 124.184314) (end 98.85 124.923654) (width 0.2) (layer "F.Cu") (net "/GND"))
 (segment (start 100 115.24) (end 102.93 118.17) (width 0.2) (layer "F.Cu") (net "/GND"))
 (segment (start 144.7 85.665685) (end 144.7 78.65) (width 0.2) (layer "F.Cu") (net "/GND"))
 (segment (start 101.09 124.25) (end 99.523654 124.25) (width 0.2) (layer "F.Cu") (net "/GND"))
 (segment (start 99.763654 126.79) (end 125.95 126.79) (width 0.2) (layer "F.Cu") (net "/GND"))
 (segment (start 98.85 128.416346) (end 99.763654 129.33) (width 0.2) (layer "F.Cu") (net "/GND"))
 (segment (start 100 115.24) (end 101.15 116.39) (width 0.2) (layer "F.Cu") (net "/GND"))
 (segment (start 101.15 124.01) (end 91.95 124.01) (width 0.2) (layer "F.Cu") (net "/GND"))
 (segment (start 98.85 124.923654) (end 98.85 125.876346) (width 0.2) (layer "F.Cu") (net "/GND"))
 (segment (start 91.825 134.498654) (end 92.6 135.273654) (width 0.2) (layer "F.Cu") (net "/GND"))
 (segment (start 105.05 117.75) (end 105.05 124.184314) (width 0.2) (layer "F.Cu") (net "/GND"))
 (segment (start 100 107.62) (end 91.825 99.445) (width 0.2) (layer "F.Cu") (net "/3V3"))
 (segment (start 90.45 77.867442) (end 92.483721 75.833721) (width 0.2) (layer "F.Cu") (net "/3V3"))
 (segment (start 92.483721 75.833721) (end 144.423721 75.833721) (width 0.2) (layer "F.Cu") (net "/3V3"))
 (segment (start 144.423721 75.833721) (end 147.24 78.65) (width 0.2) (layer "F.Cu") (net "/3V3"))
 (segment (start 90.45 98.07) (end 90.45 89.55) (width 0.2) (layer "F.Cu") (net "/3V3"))
 (segment (start 100 107.62) (end 90.45 98.07) (width 0.2) (layer "F.Cu") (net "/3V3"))
 (segment (start 90.45 89.55) (end 90.45 77.867442) (width 0.2) (layer "F.Cu") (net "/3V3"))
 (segment (start 89.775 117.845) (end 89.775 142.045) (width 0.2) (layer "F.Cu") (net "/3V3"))
 (segment (start 100 107.62) (end 89.775 117.845) (width 0.2) (layer "F.Cu") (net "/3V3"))
 (segment (start 90.45 89.55) (end 90.45 87.925) (width 0.2) (layer "F.Cu") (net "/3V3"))
 (segment (start 152.32 78.65) (end 152.32 89.34) (width 0.2) (layer "F.Cu") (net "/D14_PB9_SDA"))
 (segment (start 148.26 93.4) (end 152.32 89.34) (width 0.2) (layer "F.Cu") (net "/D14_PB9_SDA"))
 (segment (start 149.86 89.26) (end 150.01 89.11) (width 0.2) (layer "F.Cu") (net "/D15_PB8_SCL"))
 (segment (start 148.26 90.86) (end 149.86 89.26) (width 0.2) (layer "F.Cu") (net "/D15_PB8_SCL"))
 (segment (start 149.86 89.04) (end 149.78 88.96) (width 0.2) (layer "F.Cu") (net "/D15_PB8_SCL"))
 (segment (start 149.86 89.26) (end 149.86 89.04) (width 0.2) (layer "F.Cu") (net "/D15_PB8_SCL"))
 (segment (start 149.78 88.96) (end 149.78 78.65) (width 0.2) (layer "F.Cu") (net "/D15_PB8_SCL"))
 (segment (start 94.635 122.86) (end 91.425 119.65) (width 0.2) (layer "F.Cu") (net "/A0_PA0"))
 (segment (start 91.425 142.935) (end 89.775 144.585) (width 0.2) (layer "F.Cu") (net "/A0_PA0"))
 (segment (start 100 122.86) (end 94.635 122.86) (width 0.2) (layer "F.Cu") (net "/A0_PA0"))
 (segment (start 91.425 119.65) (end 91.425 142.935) (width 0.2) (layer "F.Cu") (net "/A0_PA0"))
 (segment (start 100 127.94) (end 122.24 127.94) (width 0.2) (layer "F.Cu") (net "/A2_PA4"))
 (segment (start 133 138.7) (end 133 145.525) (width 0.2) (layer "F.Cu") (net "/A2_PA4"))
 (segment (start 122.24 127.94) (end 133 138.7) (width 0.2) (layer "F.Cu") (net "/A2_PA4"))
 (segment (start 97.35 94.9) (end 92.99 90.54) (width 0.2) (layer "F.Cu") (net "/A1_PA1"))
 (segment (start 92.99 90.54) (end 92.99 87.925) (width 0.2) (layer "F.Cu") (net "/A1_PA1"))
 (segment (start 100 125.4) (end 104.1 125.4) (width 0.2) (layer "F.Cu") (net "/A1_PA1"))
 (segment (start 105.45 94.9) (end 97.35 94.9) (width 0.2) (layer "F.Cu") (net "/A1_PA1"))
 (segment (start 104.1 125.4) (end 104.25 125.55) (width 0.2) (layer "F.Cu") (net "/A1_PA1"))
 (segment (start 105.45 124.35) (end 105.45 94.9) (width 0.2) (layer "F.Cu") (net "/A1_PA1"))
 (segment (start 104.25 125.55) (end 105.45 124.35) (width 0.2) (layer "F.Cu") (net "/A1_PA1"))
 (segment (start 148.7 162.19) (end 147.85 161.34) (width 0.2) (layer "F.Cu") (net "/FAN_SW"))
 (segment (start 159.24 146.4) (end 161.3 148.46) (width 0.2) (layer "F.Cu") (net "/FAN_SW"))
 (segment (start 161.3 148.46) (end 161.3 161.232032) (width 0.2) (layer "F.Cu") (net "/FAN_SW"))
 (segment (start 161.3 161.232032) (end 160.342031 162.19) (width 0.2) (layer "F.Cu") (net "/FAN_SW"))
 (segment (start 160.342031 162.19) (end 148.7 162.19) (width 0.2) (layer "F.Cu") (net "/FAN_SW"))
 (segment (start 163.45 157.4) (end 163.45 158) (width 0.2) (layer "F.Cu") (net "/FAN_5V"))
 (segment (start 162.4 144.7) (end 163.45 145.75) (width 0.2) (layer "F.Cu") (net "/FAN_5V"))
 (segment (start 163.5 161.3) (end 163.5 163.35) (width 0.2) (layer "F.Cu") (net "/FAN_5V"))
 (segment (start 163.45 145.75) (end 163.45 157.4) (width 0.2) (layer "F.Cu") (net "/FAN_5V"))
 (segment (start 156.85 148.15) (end 156.7 148) (width 0.2) (layer "F.Cu") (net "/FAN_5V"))
 (segment (start 162.05 164.8) (end 145.1 164.8) (width 0.2) (layer "F.Cu") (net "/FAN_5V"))
 (segment (start 163.5 163.35) (end 162.05 164.8) (width 0.2) (layer "F.Cu") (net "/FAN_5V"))
 (segment (start 158.4 144.7) (end 162.4 144.7) (width 0.2) (layer "F.Cu") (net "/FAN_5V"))
 (segment (start 153.37 148.15) (end 156.85 148.15) (width 0.2) (layer "F.Cu") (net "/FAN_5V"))
 (segment (start 163.45 157.9) (end 163.5 157.9) (width 0.2) (layer "F.Cu") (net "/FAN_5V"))
 (segment (start 145.15 158.8) (end 147.85 158.8) (width 0.2) (layer "F.Cu") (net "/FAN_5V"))
 (segment (start 145.1 158.85) (end 145.15 158.8) (width 0.2) (layer "F.Cu") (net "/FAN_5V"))
 (segment (start 163.45 157.4) (end 163.45 161.25) (width 0.2) (layer "F.Cu") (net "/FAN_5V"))
 (segment (start 163.45 158) (end 163.5 158.05) (width 0.2) (layer "F.Cu") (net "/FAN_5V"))
 (segment (start 163.5 157.9) (end 163.5 158.05) (width 0.2) (layer "F.Cu") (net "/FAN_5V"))
 (segment (start 156.7 148) (end 156.7 146.4) (width 0.2) (layer "F.Cu") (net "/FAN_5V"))
 (segment (start 151.62 146.4) (end 159.75 154.53) (width 0.2) (layer "F.Cu") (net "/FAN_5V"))
 (segment (start 163.5 158.05) (end 163.5 161.3) (width 0.2) (layer "F.Cu") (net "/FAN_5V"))
 (segment (start 163.45 161.25) (end 163.5 161.3) (width 0.2) (layer "F.Cu") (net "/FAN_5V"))
 (segment (start 151.62 146.4) (end 153.37 148.15) (width 0.2) (layer "F.Cu") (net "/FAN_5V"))
 (segment (start 145.1 164.8) (end 145.1 158.85) (width 0.2) (layer "F.Cu") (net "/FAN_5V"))
 (segment (start 156.7 146.4) (end 158.4 144.7) (width 0.2) (layer "F.Cu") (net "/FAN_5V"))
 (segment (start 159.75 154.53) (end 159.75 158.05) (width 0.2) (layer "F.Cu") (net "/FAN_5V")))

